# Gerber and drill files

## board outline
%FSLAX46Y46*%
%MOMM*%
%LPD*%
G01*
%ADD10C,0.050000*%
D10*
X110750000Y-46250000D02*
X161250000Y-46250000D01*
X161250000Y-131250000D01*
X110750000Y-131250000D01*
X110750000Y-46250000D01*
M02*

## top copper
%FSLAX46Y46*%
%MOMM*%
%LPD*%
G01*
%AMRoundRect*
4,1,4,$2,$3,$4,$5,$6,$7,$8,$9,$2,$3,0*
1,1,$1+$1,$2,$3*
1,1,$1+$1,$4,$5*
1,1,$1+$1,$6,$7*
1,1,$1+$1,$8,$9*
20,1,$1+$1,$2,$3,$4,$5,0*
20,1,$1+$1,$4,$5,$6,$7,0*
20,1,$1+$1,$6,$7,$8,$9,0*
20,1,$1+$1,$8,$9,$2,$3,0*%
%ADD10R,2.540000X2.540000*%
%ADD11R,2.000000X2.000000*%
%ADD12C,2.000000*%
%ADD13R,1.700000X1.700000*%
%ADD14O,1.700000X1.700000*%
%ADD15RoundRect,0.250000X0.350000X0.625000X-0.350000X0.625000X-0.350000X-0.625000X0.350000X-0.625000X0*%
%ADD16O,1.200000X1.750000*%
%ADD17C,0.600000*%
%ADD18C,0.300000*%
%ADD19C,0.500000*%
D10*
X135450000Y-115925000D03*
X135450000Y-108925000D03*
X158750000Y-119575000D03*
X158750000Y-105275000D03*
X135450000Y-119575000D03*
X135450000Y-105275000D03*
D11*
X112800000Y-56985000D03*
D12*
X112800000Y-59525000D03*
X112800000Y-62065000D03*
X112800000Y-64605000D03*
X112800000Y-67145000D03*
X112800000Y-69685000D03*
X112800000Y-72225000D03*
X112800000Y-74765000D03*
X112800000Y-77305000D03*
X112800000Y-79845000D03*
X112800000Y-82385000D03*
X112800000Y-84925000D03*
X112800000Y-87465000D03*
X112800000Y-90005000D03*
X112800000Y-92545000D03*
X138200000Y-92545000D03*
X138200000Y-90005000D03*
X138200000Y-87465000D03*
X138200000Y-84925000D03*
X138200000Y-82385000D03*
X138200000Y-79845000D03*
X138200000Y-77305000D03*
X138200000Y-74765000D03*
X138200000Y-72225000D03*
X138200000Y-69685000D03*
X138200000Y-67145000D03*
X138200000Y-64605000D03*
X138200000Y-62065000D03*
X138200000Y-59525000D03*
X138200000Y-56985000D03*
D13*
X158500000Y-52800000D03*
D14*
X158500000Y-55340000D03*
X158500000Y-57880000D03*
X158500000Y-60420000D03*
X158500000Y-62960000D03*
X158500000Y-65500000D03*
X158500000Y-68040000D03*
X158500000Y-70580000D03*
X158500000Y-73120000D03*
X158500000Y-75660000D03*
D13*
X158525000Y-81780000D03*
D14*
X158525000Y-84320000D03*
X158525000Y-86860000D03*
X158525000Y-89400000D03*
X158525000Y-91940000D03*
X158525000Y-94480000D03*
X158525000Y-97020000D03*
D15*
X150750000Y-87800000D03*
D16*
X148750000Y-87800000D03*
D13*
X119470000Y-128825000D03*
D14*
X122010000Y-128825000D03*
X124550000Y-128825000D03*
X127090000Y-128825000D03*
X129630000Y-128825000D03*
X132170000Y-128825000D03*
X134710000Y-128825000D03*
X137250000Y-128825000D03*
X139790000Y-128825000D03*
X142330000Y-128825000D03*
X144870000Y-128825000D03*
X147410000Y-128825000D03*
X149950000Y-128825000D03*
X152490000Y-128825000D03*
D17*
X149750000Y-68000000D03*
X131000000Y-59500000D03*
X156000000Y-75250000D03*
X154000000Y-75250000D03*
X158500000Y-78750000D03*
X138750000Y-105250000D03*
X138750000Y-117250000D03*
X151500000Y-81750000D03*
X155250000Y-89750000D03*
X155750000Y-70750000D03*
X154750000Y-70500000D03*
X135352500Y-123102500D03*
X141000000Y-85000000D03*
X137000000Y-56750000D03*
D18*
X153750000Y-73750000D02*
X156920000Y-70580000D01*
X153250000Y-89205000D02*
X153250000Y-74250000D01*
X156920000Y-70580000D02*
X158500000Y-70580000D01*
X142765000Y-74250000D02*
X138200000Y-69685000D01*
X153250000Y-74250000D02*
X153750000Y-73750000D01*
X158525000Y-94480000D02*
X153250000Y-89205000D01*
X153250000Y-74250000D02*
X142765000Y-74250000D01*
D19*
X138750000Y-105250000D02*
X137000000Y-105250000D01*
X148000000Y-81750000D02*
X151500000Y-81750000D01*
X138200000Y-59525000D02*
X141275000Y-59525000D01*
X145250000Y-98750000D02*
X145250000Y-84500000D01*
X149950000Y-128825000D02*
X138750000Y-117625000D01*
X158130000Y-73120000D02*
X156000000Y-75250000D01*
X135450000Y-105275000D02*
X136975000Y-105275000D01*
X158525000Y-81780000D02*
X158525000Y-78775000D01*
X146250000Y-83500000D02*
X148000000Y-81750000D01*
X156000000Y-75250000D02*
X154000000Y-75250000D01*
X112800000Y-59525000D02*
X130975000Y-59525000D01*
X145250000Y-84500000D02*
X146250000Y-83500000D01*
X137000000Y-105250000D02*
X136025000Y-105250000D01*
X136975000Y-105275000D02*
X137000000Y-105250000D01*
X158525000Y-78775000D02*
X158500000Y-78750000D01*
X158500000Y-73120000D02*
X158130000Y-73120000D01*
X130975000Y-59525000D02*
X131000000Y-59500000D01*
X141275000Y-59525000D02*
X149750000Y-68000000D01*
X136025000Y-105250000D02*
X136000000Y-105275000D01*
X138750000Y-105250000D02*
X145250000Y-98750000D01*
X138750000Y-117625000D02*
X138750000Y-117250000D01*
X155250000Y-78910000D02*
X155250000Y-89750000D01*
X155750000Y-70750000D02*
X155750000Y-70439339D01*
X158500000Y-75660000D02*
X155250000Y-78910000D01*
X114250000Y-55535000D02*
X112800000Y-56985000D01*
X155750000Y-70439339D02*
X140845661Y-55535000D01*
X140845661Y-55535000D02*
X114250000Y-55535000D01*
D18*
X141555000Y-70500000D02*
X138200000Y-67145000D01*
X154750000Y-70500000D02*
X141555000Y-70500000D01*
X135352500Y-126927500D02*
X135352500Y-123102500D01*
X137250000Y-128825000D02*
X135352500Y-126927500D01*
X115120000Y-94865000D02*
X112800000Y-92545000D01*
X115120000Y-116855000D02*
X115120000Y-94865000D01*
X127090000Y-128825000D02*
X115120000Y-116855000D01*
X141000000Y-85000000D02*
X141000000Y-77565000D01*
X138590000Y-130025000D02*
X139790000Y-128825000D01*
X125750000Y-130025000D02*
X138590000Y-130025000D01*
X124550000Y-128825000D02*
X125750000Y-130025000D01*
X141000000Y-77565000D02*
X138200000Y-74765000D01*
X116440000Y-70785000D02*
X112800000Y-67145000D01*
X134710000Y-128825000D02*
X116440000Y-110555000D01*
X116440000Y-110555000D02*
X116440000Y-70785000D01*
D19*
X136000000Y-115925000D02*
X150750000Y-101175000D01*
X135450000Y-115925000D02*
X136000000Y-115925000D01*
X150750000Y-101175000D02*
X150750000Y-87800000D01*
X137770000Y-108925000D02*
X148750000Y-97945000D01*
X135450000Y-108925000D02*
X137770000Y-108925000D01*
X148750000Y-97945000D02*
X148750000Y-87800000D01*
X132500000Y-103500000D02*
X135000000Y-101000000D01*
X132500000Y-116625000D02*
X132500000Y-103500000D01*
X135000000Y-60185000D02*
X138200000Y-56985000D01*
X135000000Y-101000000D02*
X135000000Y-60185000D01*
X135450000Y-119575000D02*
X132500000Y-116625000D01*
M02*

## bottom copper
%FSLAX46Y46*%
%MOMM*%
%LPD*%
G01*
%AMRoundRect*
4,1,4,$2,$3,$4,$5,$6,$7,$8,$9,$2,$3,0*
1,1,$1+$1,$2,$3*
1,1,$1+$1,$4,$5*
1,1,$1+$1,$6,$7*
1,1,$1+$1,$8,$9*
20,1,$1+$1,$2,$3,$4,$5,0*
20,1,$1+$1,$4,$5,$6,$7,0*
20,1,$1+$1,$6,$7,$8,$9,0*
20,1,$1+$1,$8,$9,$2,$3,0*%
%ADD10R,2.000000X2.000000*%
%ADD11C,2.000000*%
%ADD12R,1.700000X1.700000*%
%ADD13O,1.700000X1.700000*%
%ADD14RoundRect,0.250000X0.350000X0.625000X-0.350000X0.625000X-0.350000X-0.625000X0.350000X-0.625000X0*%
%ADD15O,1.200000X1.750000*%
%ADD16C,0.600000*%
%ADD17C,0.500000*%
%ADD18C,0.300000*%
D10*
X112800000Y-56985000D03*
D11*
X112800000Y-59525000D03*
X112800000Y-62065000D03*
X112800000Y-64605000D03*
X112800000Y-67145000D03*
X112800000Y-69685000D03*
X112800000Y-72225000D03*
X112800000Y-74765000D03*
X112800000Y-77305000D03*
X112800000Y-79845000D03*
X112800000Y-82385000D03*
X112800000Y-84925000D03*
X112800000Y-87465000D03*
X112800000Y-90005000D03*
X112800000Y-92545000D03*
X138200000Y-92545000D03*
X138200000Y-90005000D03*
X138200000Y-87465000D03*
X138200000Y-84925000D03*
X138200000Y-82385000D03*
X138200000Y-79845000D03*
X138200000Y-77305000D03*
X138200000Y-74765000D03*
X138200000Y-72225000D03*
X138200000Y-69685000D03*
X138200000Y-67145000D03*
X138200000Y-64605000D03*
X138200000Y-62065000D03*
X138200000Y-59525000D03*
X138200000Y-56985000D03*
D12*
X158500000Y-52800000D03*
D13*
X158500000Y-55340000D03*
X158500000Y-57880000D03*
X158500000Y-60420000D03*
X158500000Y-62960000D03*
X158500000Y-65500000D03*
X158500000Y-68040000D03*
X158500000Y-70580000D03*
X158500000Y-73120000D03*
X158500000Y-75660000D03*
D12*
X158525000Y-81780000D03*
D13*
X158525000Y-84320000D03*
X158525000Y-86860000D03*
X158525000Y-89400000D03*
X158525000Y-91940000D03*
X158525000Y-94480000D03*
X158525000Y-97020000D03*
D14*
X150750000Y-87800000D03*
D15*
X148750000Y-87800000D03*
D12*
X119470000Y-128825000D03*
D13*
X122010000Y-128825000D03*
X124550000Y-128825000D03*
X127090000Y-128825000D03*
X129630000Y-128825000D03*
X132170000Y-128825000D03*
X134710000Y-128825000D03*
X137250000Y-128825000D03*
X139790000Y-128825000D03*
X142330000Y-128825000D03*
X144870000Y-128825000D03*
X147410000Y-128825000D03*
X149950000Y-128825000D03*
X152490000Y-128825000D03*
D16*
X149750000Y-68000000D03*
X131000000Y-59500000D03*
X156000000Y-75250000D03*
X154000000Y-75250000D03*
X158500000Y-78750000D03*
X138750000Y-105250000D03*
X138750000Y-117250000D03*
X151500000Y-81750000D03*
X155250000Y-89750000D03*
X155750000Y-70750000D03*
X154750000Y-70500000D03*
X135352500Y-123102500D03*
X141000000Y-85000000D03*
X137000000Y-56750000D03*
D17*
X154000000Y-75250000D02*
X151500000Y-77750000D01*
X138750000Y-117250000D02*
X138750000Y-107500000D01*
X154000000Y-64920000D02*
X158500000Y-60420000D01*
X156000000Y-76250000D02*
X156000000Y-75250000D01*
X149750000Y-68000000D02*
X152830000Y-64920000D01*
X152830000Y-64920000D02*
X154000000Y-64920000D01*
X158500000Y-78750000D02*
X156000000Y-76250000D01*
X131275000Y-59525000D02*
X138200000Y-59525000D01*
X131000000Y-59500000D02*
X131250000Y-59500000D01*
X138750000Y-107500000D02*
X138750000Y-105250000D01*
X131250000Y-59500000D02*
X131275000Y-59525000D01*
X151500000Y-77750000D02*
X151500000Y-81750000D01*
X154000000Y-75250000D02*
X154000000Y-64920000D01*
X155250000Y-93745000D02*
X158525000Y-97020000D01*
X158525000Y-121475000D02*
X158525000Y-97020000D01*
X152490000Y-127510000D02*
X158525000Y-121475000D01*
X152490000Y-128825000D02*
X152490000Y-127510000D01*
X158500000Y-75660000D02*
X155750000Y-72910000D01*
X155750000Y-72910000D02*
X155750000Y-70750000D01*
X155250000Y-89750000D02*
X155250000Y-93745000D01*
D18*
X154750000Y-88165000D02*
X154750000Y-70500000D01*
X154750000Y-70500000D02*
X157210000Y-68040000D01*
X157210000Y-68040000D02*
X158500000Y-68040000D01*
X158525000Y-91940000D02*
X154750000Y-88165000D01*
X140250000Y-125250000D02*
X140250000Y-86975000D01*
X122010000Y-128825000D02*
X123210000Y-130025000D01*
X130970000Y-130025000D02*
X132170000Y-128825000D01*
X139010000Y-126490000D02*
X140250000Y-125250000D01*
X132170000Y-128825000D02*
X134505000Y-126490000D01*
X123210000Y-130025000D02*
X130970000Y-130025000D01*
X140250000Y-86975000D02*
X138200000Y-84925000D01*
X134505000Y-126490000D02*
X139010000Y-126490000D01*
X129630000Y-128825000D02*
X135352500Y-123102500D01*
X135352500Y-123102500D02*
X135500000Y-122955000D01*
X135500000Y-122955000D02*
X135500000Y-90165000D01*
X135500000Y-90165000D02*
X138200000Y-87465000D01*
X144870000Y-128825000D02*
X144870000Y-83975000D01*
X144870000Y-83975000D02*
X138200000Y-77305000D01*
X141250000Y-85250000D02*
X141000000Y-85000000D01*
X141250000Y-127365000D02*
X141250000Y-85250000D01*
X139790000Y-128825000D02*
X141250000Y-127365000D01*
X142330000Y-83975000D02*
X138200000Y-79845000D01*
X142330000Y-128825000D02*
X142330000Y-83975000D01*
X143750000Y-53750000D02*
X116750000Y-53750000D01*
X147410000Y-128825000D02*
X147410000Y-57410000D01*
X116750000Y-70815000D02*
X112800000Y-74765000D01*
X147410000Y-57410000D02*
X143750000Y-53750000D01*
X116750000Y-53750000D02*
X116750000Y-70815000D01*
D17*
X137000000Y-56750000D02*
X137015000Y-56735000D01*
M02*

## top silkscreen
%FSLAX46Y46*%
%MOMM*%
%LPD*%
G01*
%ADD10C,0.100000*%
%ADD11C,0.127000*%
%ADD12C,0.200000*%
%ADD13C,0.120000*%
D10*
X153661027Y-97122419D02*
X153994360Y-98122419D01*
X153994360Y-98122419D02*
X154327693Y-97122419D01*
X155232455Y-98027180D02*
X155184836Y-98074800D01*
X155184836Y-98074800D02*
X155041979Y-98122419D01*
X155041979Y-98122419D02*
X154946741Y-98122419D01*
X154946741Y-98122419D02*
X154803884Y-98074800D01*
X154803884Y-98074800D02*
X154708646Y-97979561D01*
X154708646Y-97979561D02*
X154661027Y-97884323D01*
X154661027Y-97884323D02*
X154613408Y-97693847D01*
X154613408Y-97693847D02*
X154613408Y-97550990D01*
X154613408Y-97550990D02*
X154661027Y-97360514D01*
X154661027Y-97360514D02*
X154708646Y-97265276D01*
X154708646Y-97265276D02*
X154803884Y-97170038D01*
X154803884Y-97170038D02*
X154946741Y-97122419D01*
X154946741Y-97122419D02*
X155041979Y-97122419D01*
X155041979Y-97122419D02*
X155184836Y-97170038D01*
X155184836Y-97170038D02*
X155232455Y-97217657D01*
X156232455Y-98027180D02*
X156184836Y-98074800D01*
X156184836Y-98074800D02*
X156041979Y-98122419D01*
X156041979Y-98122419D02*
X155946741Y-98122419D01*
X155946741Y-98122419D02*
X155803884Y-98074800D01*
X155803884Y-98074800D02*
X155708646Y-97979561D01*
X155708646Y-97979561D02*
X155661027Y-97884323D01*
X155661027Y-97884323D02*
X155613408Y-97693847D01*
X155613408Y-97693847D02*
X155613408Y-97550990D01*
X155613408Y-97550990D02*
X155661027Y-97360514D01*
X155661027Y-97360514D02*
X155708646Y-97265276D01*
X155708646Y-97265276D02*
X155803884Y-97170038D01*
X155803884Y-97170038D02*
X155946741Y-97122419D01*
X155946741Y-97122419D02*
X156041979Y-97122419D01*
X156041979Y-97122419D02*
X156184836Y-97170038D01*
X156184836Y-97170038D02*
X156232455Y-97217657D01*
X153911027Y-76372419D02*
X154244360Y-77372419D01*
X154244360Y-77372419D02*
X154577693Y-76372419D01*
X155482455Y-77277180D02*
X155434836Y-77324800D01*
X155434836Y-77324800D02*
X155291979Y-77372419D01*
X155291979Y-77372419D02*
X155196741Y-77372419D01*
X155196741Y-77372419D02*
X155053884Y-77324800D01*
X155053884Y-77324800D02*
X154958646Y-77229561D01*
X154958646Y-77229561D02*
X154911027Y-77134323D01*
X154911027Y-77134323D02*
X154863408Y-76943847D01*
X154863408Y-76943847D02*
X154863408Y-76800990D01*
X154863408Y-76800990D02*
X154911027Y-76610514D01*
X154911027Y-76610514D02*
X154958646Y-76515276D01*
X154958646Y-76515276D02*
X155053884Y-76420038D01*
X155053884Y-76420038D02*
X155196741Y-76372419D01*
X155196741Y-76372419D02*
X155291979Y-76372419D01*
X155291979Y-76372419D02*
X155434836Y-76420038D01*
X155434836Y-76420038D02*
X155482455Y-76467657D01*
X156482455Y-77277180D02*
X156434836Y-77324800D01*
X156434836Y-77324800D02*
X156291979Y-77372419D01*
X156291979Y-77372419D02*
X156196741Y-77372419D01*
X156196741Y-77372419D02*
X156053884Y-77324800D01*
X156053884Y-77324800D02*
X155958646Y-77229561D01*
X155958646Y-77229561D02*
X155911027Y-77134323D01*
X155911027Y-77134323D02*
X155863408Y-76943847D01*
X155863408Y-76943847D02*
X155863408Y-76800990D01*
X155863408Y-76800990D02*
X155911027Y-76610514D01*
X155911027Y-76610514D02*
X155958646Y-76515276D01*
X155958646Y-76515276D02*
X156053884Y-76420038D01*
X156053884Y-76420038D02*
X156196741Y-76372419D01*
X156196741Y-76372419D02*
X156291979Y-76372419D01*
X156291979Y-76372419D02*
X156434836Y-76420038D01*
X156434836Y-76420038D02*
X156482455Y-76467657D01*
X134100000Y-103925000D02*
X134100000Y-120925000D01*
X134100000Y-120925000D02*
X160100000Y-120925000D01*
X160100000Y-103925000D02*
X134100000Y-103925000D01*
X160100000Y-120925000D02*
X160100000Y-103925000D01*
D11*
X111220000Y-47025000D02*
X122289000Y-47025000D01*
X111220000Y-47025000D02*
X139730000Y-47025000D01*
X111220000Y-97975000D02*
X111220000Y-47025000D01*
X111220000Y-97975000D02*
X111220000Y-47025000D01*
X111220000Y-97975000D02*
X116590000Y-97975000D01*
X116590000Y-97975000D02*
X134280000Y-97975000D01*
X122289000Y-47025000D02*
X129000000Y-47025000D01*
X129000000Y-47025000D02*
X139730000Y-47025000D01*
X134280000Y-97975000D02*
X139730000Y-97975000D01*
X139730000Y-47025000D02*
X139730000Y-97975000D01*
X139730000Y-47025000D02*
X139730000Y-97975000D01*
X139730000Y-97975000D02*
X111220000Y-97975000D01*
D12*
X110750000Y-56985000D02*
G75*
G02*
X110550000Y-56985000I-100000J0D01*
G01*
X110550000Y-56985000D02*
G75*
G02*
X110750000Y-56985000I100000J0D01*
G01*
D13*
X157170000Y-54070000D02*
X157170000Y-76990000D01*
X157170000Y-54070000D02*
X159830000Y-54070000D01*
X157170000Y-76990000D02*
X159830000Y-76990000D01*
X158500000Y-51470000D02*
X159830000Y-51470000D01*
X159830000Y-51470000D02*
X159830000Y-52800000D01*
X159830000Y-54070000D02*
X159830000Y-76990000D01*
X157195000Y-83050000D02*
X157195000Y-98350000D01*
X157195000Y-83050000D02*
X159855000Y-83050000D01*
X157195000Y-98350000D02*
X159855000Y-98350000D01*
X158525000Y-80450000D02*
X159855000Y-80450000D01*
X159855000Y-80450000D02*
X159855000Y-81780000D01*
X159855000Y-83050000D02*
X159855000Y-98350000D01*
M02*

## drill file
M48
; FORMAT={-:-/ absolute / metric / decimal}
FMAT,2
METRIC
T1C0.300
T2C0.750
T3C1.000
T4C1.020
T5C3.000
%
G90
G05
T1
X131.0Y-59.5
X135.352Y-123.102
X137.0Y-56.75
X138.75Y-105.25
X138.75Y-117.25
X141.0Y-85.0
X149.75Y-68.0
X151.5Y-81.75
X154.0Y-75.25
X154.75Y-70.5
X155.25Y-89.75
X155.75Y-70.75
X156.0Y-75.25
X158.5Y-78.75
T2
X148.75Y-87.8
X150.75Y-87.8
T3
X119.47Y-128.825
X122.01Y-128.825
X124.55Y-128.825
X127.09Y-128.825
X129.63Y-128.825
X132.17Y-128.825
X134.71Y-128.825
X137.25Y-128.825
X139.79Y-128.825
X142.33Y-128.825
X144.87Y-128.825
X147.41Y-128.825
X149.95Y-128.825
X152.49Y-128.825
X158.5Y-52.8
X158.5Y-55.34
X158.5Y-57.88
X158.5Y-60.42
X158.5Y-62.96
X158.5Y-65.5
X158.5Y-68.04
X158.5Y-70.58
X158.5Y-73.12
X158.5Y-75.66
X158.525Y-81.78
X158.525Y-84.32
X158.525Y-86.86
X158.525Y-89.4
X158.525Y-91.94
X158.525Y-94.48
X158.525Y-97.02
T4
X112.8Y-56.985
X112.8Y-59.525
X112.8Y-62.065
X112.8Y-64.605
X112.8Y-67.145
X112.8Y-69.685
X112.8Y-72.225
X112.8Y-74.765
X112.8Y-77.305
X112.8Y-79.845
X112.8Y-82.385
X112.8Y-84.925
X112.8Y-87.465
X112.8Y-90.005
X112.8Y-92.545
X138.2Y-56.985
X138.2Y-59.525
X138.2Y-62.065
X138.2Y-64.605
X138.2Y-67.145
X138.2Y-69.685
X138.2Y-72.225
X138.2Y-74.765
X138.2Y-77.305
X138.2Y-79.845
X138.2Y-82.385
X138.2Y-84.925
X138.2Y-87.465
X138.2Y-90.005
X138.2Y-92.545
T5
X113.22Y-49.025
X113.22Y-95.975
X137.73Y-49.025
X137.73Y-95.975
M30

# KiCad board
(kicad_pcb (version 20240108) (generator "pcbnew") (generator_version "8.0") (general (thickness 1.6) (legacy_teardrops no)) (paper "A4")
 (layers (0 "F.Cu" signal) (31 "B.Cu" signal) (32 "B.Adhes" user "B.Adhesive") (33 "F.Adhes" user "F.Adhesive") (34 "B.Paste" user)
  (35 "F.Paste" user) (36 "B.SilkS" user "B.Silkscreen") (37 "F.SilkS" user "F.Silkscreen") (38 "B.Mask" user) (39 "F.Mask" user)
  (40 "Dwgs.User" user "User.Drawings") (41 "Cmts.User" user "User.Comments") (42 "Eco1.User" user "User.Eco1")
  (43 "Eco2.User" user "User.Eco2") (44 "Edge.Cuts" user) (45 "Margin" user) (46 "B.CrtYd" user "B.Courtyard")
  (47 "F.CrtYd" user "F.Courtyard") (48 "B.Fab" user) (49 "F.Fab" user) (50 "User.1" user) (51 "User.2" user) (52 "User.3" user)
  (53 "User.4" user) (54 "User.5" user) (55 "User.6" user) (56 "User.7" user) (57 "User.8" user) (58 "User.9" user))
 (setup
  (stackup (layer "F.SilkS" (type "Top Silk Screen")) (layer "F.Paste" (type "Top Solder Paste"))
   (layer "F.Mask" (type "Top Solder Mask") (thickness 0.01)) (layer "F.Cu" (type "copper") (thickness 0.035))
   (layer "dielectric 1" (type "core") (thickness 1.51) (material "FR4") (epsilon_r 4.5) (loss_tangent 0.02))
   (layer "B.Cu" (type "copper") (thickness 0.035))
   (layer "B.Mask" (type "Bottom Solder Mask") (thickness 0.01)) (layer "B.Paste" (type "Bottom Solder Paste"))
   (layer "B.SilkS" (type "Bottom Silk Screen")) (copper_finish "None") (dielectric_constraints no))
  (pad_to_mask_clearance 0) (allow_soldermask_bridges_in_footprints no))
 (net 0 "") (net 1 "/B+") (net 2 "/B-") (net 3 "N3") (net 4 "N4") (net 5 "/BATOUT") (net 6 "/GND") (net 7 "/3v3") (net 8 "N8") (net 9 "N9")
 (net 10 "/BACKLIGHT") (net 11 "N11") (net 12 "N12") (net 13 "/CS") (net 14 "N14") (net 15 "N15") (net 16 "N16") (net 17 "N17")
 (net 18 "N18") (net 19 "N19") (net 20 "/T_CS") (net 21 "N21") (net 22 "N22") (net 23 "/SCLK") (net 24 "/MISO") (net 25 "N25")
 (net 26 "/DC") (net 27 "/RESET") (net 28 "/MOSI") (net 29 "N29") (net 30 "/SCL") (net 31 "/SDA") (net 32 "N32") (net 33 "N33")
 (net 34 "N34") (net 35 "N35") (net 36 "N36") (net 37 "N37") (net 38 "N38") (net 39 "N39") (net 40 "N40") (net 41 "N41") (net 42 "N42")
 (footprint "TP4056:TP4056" (layer "F.Cu") (at 134.1 103.925 -90)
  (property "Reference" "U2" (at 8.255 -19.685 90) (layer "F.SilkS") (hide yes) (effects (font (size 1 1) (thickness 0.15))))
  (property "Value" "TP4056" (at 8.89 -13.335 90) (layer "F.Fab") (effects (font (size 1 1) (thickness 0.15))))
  (fp_line (start 0 0) (end 17 0) (stroke (width 0.1) (type solid)) (layer "F.SilkS"))
  (fp_line (start 17 0) (end 17 -26) (stroke (width 0.1) (type solid)) (layer "F.SilkS"))
  (fp_line (start 0 -26) (end 0 0) (stroke (width 0.1) (type solid)) (layer "F.SilkS"))
  (fp_line (start 17 -26) (end 0 -26) (stroke (width 0.1) (type solid)) (layer "F.SilkS"))
  (pad "B+" smd rect (at 12 -1.35 270) (size 2.54 2.54) (layers "F.Cu" "F.Paste" "F.Mask") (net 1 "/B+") (solder_mask_margin 0.102))
  (pad "B-" smd rect (at 5 -1.35 270) (size 2.54 2.54) (layers "F.Cu" "F.Paste" "F.Mask") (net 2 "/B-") (solder_mask_margin 0.102))
  (pad "IN+" smd rect (at 15.65 -24.65 270) (size 2.54 2.54) (layers "F.Cu" "F.Paste" "F.Mask") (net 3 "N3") (solder_mask_margin 0.102))
  (pad "IN-" smd rect (at 1.35 -24.65 270) (size 2.54 2.54) (layers "F.Cu" "F.Paste" "F.Mask") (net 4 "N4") (solder_mask_margin 0.102))
  (pad "OUT+" smd rect (at 15.65 -1.35 270) (size 2.54 2.54) (layers "F.Cu" "F.Paste" "F.Mask") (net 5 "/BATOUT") (solder_mask_margin 0.102))
  (pad "OUT-" smd rect (at 1.35 -1.35 270) (size 2.54 2.54) (layers "F.Cu" "F.Paste" "F.Mask") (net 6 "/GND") (solder_mask_margin 0.102)))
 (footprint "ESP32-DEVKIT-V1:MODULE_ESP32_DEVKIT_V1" (layer "F.Cu") (at 125.5 72.5)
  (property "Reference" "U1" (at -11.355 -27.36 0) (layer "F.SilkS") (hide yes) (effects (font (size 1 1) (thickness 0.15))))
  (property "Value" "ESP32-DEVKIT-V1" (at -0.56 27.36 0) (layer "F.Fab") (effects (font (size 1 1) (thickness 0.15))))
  (fp_line (start -14.28 -25.475) (end -3.211 -25.475) (stroke (width 0.127) (type solid)) (layer "F.SilkS"))
  (fp_line (start -14.28 -25.475) (end 14.23 -25.475) (stroke (width 0.127) (type solid)) (layer "F.SilkS"))
  (fp_line (start -14.28 25.475) (end -14.28 -25.475) (stroke (width 0.127) (type solid)) (layer "F.SilkS"))
  (fp_line (start -14.28 25.475) (end -14.28 -25.475) (stroke (width 0.127) (type solid)) (layer "F.SilkS"))
  (fp_line (start -14.28 25.475) (end -8.91 25.475) (stroke (width 0.127) (type solid)) (layer "F.SilkS"))
  (fp_line (start -8.91 25.475) (end 8.78 25.475) (stroke (width 0.127) (type solid)) (layer "F.SilkS"))
  (fp_line (start -3.211 -25.475) (end 3.5 -25.475) (stroke (width 0.127) (type solid)) (layer "F.SilkS"))
  (fp_line (start 3.5 -25.475) (end 14.23 -25.475) (stroke (width 0.127) (type solid)) (layer "F.SilkS"))
  (fp_line (start 8.78 25.475) (end 14.23 25.475) (stroke (width 0.127) (type solid)) (layer "F.SilkS"))
  (fp_line (start 14.23 -25.475) (end 14.23 25.475) (stroke (width 0.127) (type solid)) (layer "F.SilkS"))
  (fp_line (start 14.23 -25.475) (end 14.23 25.475) (stroke (width 0.127) (type solid)) (layer "F.SilkS"))
  (fp_line (start 14.23 25.475) (end -14.28 25.475) (stroke (width 0.127) (type solid)) (layer "F.SilkS"))
  (fp_circle (center -14.85 -15.515) (end -14.75 -15.515) (stroke (width 0.2) (type solid)) (fill none) (layer "F.SilkS"))
  (pad "" np_thru_hole circle (at -12.28 -23.475) (size 3 3) (drill 3) (layers "*.Cu" "*.Mask"))
  (pad "" np_thru_hole circle (at -12.28 23.475) (size 3 3) (drill 3) (layers "*.Cu" "*.Mask"))
  (pad "" np_thru_hole circle (at 12.23 -23.475) (size 3 3) (drill 3) (layers "*.Cu" "*.Mask"))
  (pad "" np_thru_hole circle (at 12.23 23.475) (size 3 3) (drill 3) (layers "*.Cu" "*.Mask"))
  (pad "1" thru_hole rect (at -12.7 -15.515) (size 2 2) (drill 1.02) (layers "*.Cu" "*.Mask") (remove_unused_layers no) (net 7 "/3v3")
   (solder_mask_margin 0.102))
  (pad "2" thru_hole circle (at -12.7 -12.975) (size 2 2) (drill 1.02) (layers "*.Cu" "*.Mask") (remove_unused_layers no) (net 6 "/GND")
   (solder_mask_margin 0.102))
  (pad "3" thru_hole circle (at -12.7 -10.435) (size 2 2) (drill 1.02) (layers "*.Cu" "*.Mask") (remove_unused_layers no) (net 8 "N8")
   (solder_mask_margin 0.102))
  (pad "4" thru_hole circle (at -12.7 -7.895) (size 2 2) (drill 1.02) (layers "*.Cu" "*.Mask") (remove_unused_layers no) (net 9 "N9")
   (solder_mask_margin 0.102))
  (pad "5" thru_hole circle (at -12.7 -5.355) (size 2 2) (drill 1.02) (layers "*.Cu" "*.Mask") (remove_unused_layers no)
   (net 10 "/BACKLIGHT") (solder_mask_margin 0.102))
  (pad "6" thru_hole circle (at -12.7 -2.815) (size 2 2) (drill 1.02) (layers "*.Cu" "*.Mask") (remove_unused_layers no) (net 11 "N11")
   (solder_mask_margin 0.102))
  (pad "7" thru_hole circle (at -12.7 -0.275) (size 2 2) (drill 1.02) (layers "*.Cu" "*.Mask") (remove_unused_layers no) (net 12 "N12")
   (solder_mask_margin 0.102))
  (pad "8" thru_hole circle (at -12.7 2.265) (size 2 2) (drill 1.02) (layers "*.Cu" "*.Mask") (remove_unused_layers no) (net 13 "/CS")
   (solder_mask_margin 0.102))
  (pad "9" thru_hole circle (at -12.7 4.805) (size 2 2) (drill 1.02) (layers "*.Cu" "*.Mask") (remove_unused_layers no) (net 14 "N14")
   (solder_mask_margin 0.102))
  (pad "10" thru_hole circle (at -12.7 7.345) (size 2 2) (drill 1.02) (layers "*.Cu" "*.Mask") (remove_unused_layers no) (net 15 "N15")
   (solder_mask_margin 0.102))
  (pad "11" thru_hole circle (at -12.7 9.885) (size 2 2) (drill 1.02) (layers "*.Cu" "*.Mask") (remove_unused_layers no) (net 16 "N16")
   (solder_mask_margin 0.102))
  (pad "12" thru_hole circle (at -12.7 12.425) (size 2 2) (drill 1.02) (layers "*.Cu" "*.Mask") (remove_unused_layers no) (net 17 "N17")
   (solder_mask_margin 0.102))
  (pad "13" thru_hole circle (at -12.7 14.965) (size 2 2) (drill 1.02) (layers "*.Cu" "*.Mask") (remove_unused_layers no) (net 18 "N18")
   (solder_mask_margin 0.102))
  (pad "14" thru_hole circle (at -12.7 17.505) (size 2 2) (drill 1.02) (layers "*.Cu" "*.Mask") (remove_unused_layers no) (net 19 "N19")
   (solder_mask_margin 0.102))
  (pad "15" thru_hole circle (at -12.7 20.045) (size 2 2) (drill 1.02) (layers "*.Cu" "*.Mask") (remove_unused_layers no) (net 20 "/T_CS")
   (solder_mask_margin 0.102))
  (pad "16" thru_hole circle (at 12.7 20.045) (size 2 2) (drill 1.02) (layers "*.Cu" "*.Mask") (remove_unused_layers no) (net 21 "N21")
   (solder_mask_margin 0.102))
  (pad "17" thru_hole circle (at 12.7 17.505) (size 2 2) (drill 1.02) (layers "*.Cu" "*.Mask") (remove_unused_layers no) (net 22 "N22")
   (solder_mask_margin 0.102))
  (pad "18" thru_hole circle (at 12.7 14.965) (size 2 2) (drill 1.02) (layers "*.Cu" "*.Mask") (remove_unused_layers no) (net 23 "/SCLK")
   (solder_mask_margin 0.102))
  (pad "19" thru_hole circle (at 12.7 12.425) (size 2 2) (drill 1.02) (layers "*.Cu" "*.Mask") (remove_unused_layers no) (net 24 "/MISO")
   (solder_mask_margin 0.102))
  (pad "20" thru_hole circle (at 12.7 9.885) (size 2 2) (drill 1.02) (layers "*.Cu" "*.Mask") (remove_unused_layers no) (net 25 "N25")
   (solder_mask_margin 0.102))
  (pad "21" thru_hole circle (at 12.7 7.345) (size 2 2) (drill 1.02) (layers "*.Cu" "*.Mask") (remove_unused_layers no) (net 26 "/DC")
   (solder_mask_margin 0.102))
  (pad "22" thru_hole circle (at 12.7 4.805) (size 2 2) (drill 1.02) (layers "*.Cu" "*.Mask") (remove_unused_layers no) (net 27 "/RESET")
   (solder_mask_margin 0.102))
  (pad "23" thru_hole circle (at 12.7 2.265) (size 2 2) (drill 1.02) (layers "*.Cu" "*.Mask") (remove_unused_layers no) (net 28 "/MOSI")
   (solder_mask_margin 0.102))
  (pad "24" thru_hole circle (at 12.7 -0.275) (size 2 2) (drill 1.02) (layers "*.Cu" "*.Mask") (remove_unused_layers no) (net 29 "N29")
   (solder_mask_margin 0.102))
  (pad "25" thru_hole circle (at 12.7 -2.815) (size 2 2) (drill 1.02) (layers "*.Cu" "*.Mask") (remove_unused_layers no) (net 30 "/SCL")
   (solder_mask_margin 0.102))
  (pad "26" thru_hole circle (at 12.7 -5.355) (size 2 2) (drill 1.02) (layers "*.Cu" "*.Mask") (remove_unused_layers no) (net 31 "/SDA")
   (solder_mask_margin 0.102))
  (pad "27" thru_hole circle (at 12.7 -7.895) (size 2 2) (drill 1.02) (layers "*.Cu" "*.Mask") (remove_unused_layers no) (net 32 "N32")
   (solder_mask_margin 0.102))
  (pad "28" thru_hole circle (at 12.7 -10.435) (size 2 2) (drill 1.02) (layers "*.Cu" "*.Mask") (remove_unused_layers no) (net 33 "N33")
   (solder_mask_margin 0.102))
  (pad "29" thru_hole circle (at 12.7 -12.975) (size 2 2) (drill 1.02) (layers "*.Cu" "*.Mask") (remove_unused_layers no) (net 6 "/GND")
   (solder_mask_margin 0.102))
  (pad "30" thru_hole circle (at 12.7 -15.515) (size 2 2) (drill 1.02) (layers "*.Cu" "*.Mask") (remove_unused_layers no) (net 5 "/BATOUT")
   (solder_mask_margin 0.102))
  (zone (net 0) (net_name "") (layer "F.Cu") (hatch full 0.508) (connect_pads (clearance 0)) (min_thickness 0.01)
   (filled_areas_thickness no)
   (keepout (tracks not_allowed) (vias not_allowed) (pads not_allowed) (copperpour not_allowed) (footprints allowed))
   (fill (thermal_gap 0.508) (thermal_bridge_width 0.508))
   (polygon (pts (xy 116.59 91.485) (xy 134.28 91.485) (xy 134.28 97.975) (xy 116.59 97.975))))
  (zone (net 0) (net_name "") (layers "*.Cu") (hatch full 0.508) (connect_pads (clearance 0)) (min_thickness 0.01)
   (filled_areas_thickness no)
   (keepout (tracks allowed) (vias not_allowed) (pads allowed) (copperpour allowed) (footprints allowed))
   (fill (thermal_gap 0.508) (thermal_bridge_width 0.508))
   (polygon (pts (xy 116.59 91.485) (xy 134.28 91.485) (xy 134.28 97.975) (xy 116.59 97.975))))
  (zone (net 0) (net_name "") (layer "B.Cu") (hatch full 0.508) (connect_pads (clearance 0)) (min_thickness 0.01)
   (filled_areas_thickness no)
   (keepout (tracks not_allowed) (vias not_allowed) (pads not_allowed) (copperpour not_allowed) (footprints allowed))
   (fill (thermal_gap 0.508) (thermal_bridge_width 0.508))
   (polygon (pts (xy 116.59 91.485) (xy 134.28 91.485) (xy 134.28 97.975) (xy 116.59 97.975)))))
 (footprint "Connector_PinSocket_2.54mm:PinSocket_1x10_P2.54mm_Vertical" (layer "F.Cu") (at 158.5 52.8)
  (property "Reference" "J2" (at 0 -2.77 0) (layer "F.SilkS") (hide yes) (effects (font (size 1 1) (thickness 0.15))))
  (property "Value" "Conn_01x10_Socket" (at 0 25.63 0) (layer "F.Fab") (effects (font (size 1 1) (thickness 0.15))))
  (fp_line (start -1.33 1.27) (end -1.33 24.19) (stroke (width 0.12) (type solid)) (layer "F.SilkS"))
  (fp_line (start -1.33 1.27) (end 1.33 1.27) (stroke (width 0.12) (type solid)) (layer "F.SilkS"))
  (fp_line (start -1.33 24.19) (end 1.33 24.19) (stroke (width 0.12) (type solid)) (layer "F.SilkS"))
  (fp_line (start 0 -1.33) (end 1.33 -1.33) (stroke (width 0.12) (type solid)) (layer "F.SilkS"))
  (fp_line (start 1.33 -1.33) (end 1.33 0) (stroke (width 0.12) (type solid)) (layer "F.SilkS"))
  (fp_line (start 1.33 1.27) (end 1.33 24.19) (stroke (width 0.12) (type solid)) (layer "F.SilkS"))
  (pad "1" thru_hole rect (at 0 0) (size 1.7 1.7) (drill 1) (layers "*.Cu" "*.Mask") (remove_unused_layers no) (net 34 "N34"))
  (pad "2" thru_hole oval (at 0 2.54) (size 1.7 1.7) (drill 1) (layers "*.Cu" "*.Mask") (remove_unused_layers no) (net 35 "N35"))
  (pad "3" thru_hole oval (at 0 5.08) (size 1.7 1.7) (drill 1) (layers "*.Cu" "*.Mask") (remove_unused_layers no) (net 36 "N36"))
  (pad "4" thru_hole oval (at 0 7.62) (size 1.7 1.7) (drill 1) (layers "*.Cu" "*.Mask") (remove_unused_layers no) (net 6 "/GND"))
  (pad "5" thru_hole oval (at 0 10.16) (size 1.7 1.7) (drill 1) (layers "*.Cu" "*.Mask") (remove_unused_layers no) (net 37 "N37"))
  (pad "6" thru_hole oval (at 0 12.7) (size 1.7 1.7) (drill 1) (layers "*.Cu" "*.Mask") (remove_unused_layers no) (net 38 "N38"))
  (pad "7" thru_hole oval (at 0 15.24) (size 1.7 1.7) (drill 1) (layers "*.Cu" "*.Mask") (remove_unused_layers no) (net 31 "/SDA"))
  (pad "8" thru_hole oval (at 0 17.78) (size 1.7 1.7) (drill 1) (layers "*.Cu" "*.Mask") (remove_unused_layers no) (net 30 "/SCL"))
  (pad "9" thru_hole oval (at 0 20.32) (size 1.7 1.7) (drill 1) (layers "*.Cu" "*.Mask") (remove_unused_layers no) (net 6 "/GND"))
  (pad "10" thru_hole oval (at 0 22.86) (size 1.7 1.7) (drill 1) (layers "*.Cu" "*.Mask") (remove_unused_layers no) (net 7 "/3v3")))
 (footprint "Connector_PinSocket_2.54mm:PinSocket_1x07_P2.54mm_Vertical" (layer "F.Cu") (at 158.525 81.78)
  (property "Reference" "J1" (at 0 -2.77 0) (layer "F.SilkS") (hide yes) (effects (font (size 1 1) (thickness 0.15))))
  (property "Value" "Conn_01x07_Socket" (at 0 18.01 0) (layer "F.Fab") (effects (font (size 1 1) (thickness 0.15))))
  (fp_line (start -1.33 1.27) (end -1.33 16.57) (stroke (width 0.12) (type solid)) (layer "F.SilkS"))
  (fp_line (start -1.33 1.27) (end 1.33 1.27) (stroke (width 0.12) (type solid)) (layer "F.SilkS"))
  (fp_line (start -1.33 16.57) (end 1.33 16.57) (stroke (width 0.12) (type solid)) (layer "F.SilkS"))
  (fp_line (start 0 -1.33) (end 1.33 -1.33) (stroke (width 0.12) (type solid)) (layer "F.SilkS"))
  (fp_line (start 1.33 -1.33) (end 1.33 0) (stroke (width 0.12) (type solid)) (layer "F.SilkS"))
  (fp_line (start 1.33 1.27) (end 1.33 16.57) (stroke (width 0.12) (type solid)) (layer "F.SilkS"))
  (pad "1" thru_hole rect (at 0 0) (size 1.7 1.7) (drill 1) (layers "*.Cu" "*.Mask") (remove_unused_layers no) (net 6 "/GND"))
  (pad "2" thru_hole oval (at 0 2.54) (size 1.7 1.7) (drill 1) (layers "*.Cu" "*.Mask") (remove_unused_layers no) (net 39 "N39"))
  (pad "3" thru_hole oval (at 0 5.08) (size 1.7 1.7) (drill 1) (layers "*.Cu" "*.Mask") (remove_unused_layers no) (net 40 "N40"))
  (pad "4" thru_hole oval (at 0 7.62) (size 1.7 1.7) (drill 1) (layers "*.Cu" "*.Mask") (remove_unused_layers no) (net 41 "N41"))
  (pad "5" thru_hole oval (at 0 10.16) (size 1.7 1.7) (drill 1) (layers "*.Cu" "*.Mask") (remove_unused_layers no) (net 31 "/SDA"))
  (pad "6" thru_hole oval (at 0 12.7) (size 1.7 1.7) (drill 1) (layers "*.Cu" "*.Mask") (remove_unused_layers no) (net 30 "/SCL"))
  (pad "7" thru_hole oval (at 0 15.24) (size 1.7 1.7) (drill 1) (layers "*.Cu" "*.Mask") (remove_unused_layers no) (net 7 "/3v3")))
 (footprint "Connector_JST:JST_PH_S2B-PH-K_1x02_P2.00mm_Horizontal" (layer "B.Cu") (at 150.75 87.8 180)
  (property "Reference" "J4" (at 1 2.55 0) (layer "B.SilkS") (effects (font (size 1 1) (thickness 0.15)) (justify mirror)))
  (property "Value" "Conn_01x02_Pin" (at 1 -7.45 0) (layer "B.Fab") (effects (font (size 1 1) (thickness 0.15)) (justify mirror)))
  (pad "1" thru_hole roundrect (at 0 0 180) (size 1.2 1.75) (drill 0.75) (layers "*.Cu" "*.Mask") (remove_unused_layers no)
   (roundrect_rratio 0.208333) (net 1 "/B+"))
  (pad "2" thru_hole oval (at 2 0 180) (size 1.2 1.75) (drill 0.75) (layers "*.Cu" "*.Mask") (remove_unused_layers no) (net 2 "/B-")))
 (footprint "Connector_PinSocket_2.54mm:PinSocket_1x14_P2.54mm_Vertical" (layer "B.Cu") (at 119.47 128.825 -90)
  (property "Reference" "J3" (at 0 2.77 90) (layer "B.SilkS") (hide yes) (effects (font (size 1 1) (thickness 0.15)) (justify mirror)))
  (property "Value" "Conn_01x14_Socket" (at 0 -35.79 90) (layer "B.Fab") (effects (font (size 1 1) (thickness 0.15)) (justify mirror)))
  (pad "1" thru_hole rect (at 0 0 270) (size 1.7 1.7) (drill 1) (layers "*.Cu" "*.Mask") (remove_unused_layers no) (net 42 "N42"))
  (pad "2" thru_hole oval (at 0 -2.54 270) (size 1.7 1.7) (drill 1) (layers "*.Cu" "*.Mask") (remove_unused_layers no) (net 24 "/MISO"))
  (pad "3" thru_hole oval (at 0 -5.08 270) (size 1.7 1.7) (drill 1) (layers "*.Cu" "*.Mask") (remove_unused_layers no) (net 28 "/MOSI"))
  (pad "4" thru_hole oval (at 0 -7.62 270) (size 1.7 1.7) (drill 1) (layers "*.Cu" "*.Mask") (remove_unused_layers no) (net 20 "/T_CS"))
  (pad "5" thru_hole oval (at 0 -10.16 270) (size 1.7 1.7) (drill 1) (layers "*.Cu" "*.Mask") (remove_unused_layers no) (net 23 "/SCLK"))
  (pad "6" thru_hole oval (at 0 -12.7 270) (size 1.7 1.7) (drill 1) (layers "*.Cu" "*.Mask") (remove_unused_layers no) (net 24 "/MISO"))
  (pad "7" thru_hole oval (at 0 -15.24 270) (size 1.7 1.7) (drill 1) (layers "*.Cu" "*.Mask") (remove_unused_layers no)
   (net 10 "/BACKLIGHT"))
  (pad "8" thru_hole oval (at 0 -17.78 270) (size 1.7 1.7) (drill 1) (layers "*.Cu" "*.Mask") (remove_unused_layers no) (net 23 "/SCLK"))
  (pad "9" thru_hole oval (at 0 -20.32 270) (size 1.7 1.7) (drill 1) (layers "*.Cu" "*.Mask") (remove_unused_layers no) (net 28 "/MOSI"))
  (pad "10" thru_hole oval (at 0 -22.86 270) (size 1.7 1.7) (drill 1) (layers "*.Cu" "*.Mask") (remove_unused_layers no) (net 26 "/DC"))
  (pad "11" thru_hole oval (at 0 -25.4 270) (size 1.7 1.7) (drill 1) (layers "*.Cu" "*.Mask") (remove_unused_layers no) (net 27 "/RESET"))
  (pad "12" thru_hole oval (at 0 -27.94 270) (size 1.7 1.7) (drill 1) (layers "*.Cu" "*.Mask") (remove_unused_layers no) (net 13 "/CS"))
  (pad "13" thru_hole oval (at 0 -30.48 270) (size 1.7 1.7) (drill 1) (layers "*.Cu" "*.Mask") (remove_unused_layers no) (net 6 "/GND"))
  (pad "14" thru_hole oval (at 0 -33.02 270) (size 1.7 1.7) (drill 1) (layers "*.Cu" "*.Mask") (remove_unused_layers no) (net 7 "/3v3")))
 (gr_rect (start 110.75 46.25) (end 161.25 131.25) (stroke (width 0.05) (type default)) (fill none) (layer "Edge.Cuts"))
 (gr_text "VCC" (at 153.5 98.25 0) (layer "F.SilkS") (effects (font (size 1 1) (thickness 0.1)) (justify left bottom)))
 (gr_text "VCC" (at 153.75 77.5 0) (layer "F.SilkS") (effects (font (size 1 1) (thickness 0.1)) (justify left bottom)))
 (segment (start 153.75 73.75) (end 156.92 70.58) (width 0.3) (layer "F.Cu") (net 30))
 (segment (start 153.25 89.205) (end 153.25 74.25) (width 0.3) (layer "F.Cu") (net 30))
 (segment (start 156.92 70.58) (end 158.5 70.58) (width 0.3) (layer "F.Cu") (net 30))
 (segment (start 142.765 74.25) (end 138.2 69.685) (width 0.3) (layer "F.Cu") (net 30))
 (segment (start 153.25 74.25) (end 153.75 73.75) (width 0.3) (layer "F.Cu") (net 30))
 (segment (start 158.525 94.48) (end 153.25 89.205) (width 0.3) (layer "F.Cu") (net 30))
 (segment (start 153.25 74.25) (end 142.765 74.25) (width 0.3) (layer "F.Cu") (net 30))
 (segment (start 138.75 105.25) (end 137 105.25) (width 0.5) (layer "F.Cu") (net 6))
 (segment (start 148 81.75) (end 151.5 81.75) (width 0.5) (layer "F.Cu") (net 6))
 (segment (start 138.2 59.525) (end 141.275 59.525) (width 0.5) (layer "F.Cu") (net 6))
 (segment (start 145.25 98.75) (end 145.25 84.5) (width 0.5) (layer "F.Cu") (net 6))
 (segment (start 149.95 128.825) (end 138.75 117.625) (width 0.5) (layer "F.Cu") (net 6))
 (segment (start 158.13 73.12) (end 156 75.25) (width 0.5) (layer "F.Cu") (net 6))
 (segment (start 135.45 105.275) (end 136.975 105.275) (width 0.5) (layer "F.Cu") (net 6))
 (segment (start 158.525 81.78) (end 158.525 78.775) (width 0.5) (layer "F.Cu") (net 6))
 (segment (start 146.25 83.5) (end 148 81.75) (width 0.5) (layer "F.Cu") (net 6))
 (segment (start 156 75.25) (end 154 75.25) (width 0.5) (layer "F.Cu") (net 6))
 (segment (start 112.8 59.525) (end 130.975 59.525) (width 0.5) (layer "F.Cu") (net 6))
 (segment (start 145.25 84.5) (end 146.25 83.5) (width 0.5) (layer "F.Cu") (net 6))
 (segment (start 137 105.25) (end 136.025 105.25) (width 0.5) (layer "F.Cu") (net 6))
 (segment (start 136.975 105.275) (end 137 105.25) (width 0.5) (layer "F.Cu") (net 6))
 (segment (start 158.525 78.775) (end 158.5 78.75) (width 0.5) (layer "F.Cu") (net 6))
 (segment (start 158.5 73.12) (end 158.13 73.12) (width 0.5) (layer "F.Cu") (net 6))
 (segment (start 130.975 59.525) (end 131 59.5) (width 0.5) (layer "F.Cu") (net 6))
 (segment (start 141.275 59.525) (end 149.75 68) (width 0.5) (layer "F.Cu") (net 6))
 (segment (start 136.025 105.25) (end 136 105.275) (width 0.5) (layer "F.Cu") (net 6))
 (segment (start 138.75 105.25) (end 145.25 98.75) (width 0.5) (layer "F.Cu") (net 6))
 (segment (start 138.75 117.625) (end 138.75 117.25) (width 0.5) (layer "F.Cu") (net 6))
 (via (at 149.75 68) (size 0.6) (drill 0.3) (layers "F.Cu" "B.Cu") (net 6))
 (via (at 131 59.5) (size 0.6) (drill 0.3) (layers "F.Cu" "B.Cu") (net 6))
 (via (at 156 75.25) (size 0.6) (drill 0.3) (layers "F.Cu" "B.Cu") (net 6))
 (via (at 154 75.25) (size 0.6) (drill 0.3) (layers "F.Cu" "B.Cu") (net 6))
 (via (at 158.5 78.75) (size 0.6) (drill 0.3) (layers "F.Cu" "B.Cu") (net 6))
 (via (at 138.75 105.25) (size 0.6) (drill 0.3) (layers "F.Cu" "B.Cu") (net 6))
 (via (at 138.75 117.25) (size 0.6) (drill 0.3) (layers "F.Cu" "B.Cu") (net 6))
 (via (at 151.5 81.75) (size 0.6) (drill 0.3) (layers "F.Cu" "B.Cu") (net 6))
 (segment (start 154 75.25) (end 151.5 77.75) (width 0.5) (layer "B.Cu") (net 6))
 (segment (start 138.75 117.25) (end 138.75 107.5) (width 0.5) (layer "B.Cu") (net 6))
 (segment (start 154 64.92) (end 158.5 60.42) (width 0.5) (layer "B.Cu") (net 6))
 (segment (start 156 76.25) (end 156 75.25) (width 0.5) (layer "B.Cu") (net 6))
 (segment (start 149.75 68) (end 152.83 64.92) (width 0.5) (layer "B.Cu") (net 6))
 (segment (start 152.83 64.92) (end 154 64.92) (width 0.5) (layer "B.Cu") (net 6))
 (segment (start 158.5 78.75) (end 156 76.25) (width 0.5) (layer "B.Cu") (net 6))
 (segment (start 131.275 59.525) (end 138.2 59.525) (width 0.5) (layer "B.Cu") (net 6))
 (segment (start 131 59.5) (end 131.25 59.5) (width 0.5) (layer "B.Cu") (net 6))
 (segment (start 138.75 107.5) (end 138.75 105.25) (width 0.5) (layer "B.Cu") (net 6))
 (segment (start 131.25 59.5) (end 131.275 59.525) (width 0.5) (layer "B.Cu") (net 6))
 (segment (start 151.5 77.75) (end 151.5 81.75) (width 0.5) (layer "B.Cu") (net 6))
 (segment (start 154 75.25) (end 154 64.92) (width 0.5) (layer "B.Cu") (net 6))
 (segment (start 155.25 78.91) (end 155.25 89.75) (width 0.5) (layer "F.Cu") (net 7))
 (segment (start 155.75 70.75) (end 155.75 70.439339) (width 0.5) (layer "F.Cu") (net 7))
 (segment (start 158.5 75.66) (end 155.25 78.91) (width 0.5) (layer "F.Cu") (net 7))
 (segment (start 114.25 55.535) (end 112.8 56.985) (width 0.5) (layer "F.Cu") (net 7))
 (segment (start 155.75 70.439339) (end 140.845661 55.535) (width 0.5) (layer "F.Cu") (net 7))
 (segment (start 140.845661 55.535) (end 114.25 55.535) (width 0.5) (layer "F.Cu") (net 7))
 (via (at 155.25 89.75) (size 0.6) (drill 0.3) (layers "F.Cu" "B.Cu") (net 7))
 (via (at 155.75 70.75) (size 0.6) (drill 0.3) (layers "F.Cu" "B.Cu") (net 7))
 (segment (start 155.25 93.745) (end 158.525 97.02) (width 0.5) (layer "B.Cu") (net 7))
 (segment (start 158.525 121.475) (end 158.525 97.02) (width 0.5) (layer "B.Cu") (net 7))
 (segment (start 152.49 127.51) (end 158.525 121.475) (width 0.5) (layer "B.Cu") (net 7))
 (segment (start 152.49 128.825) (end 152.49 127.51) (width 0.5) (layer "B.Cu") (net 7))
 (segment (start 158.5 75.66) (end 155.75 72.91) (width 0.5) (layer "B.Cu") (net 7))
 (segment (start 155.75 72.91) (end 155.75 70.75) (width 0.5) (layer "B.Cu") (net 7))
 (segment (start 155.25 89.75) (end 155.25 93.745) (width 0.5) (layer "B.Cu") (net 7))
 (segment (start 141.555 70.5) (end 138.2 67.145) (width 0.3) (layer "F.Cu") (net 31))
 (segment (start 154.75 70.5) (end 141.555 70.5) (width 0.3) (layer "F.Cu") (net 31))
 (via (at 154.75 70.5) (size 0.6) (drill 0.3) (layers "F.Cu" "B.Cu") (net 31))
 (segment (start 154.75 88.165) (end 154.75 70.5) (width 0.3) (layer "B.Cu") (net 31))
 (segment (start 154.75 70.5) (end 157.21 68.04) (width 0.3) (layer "B.Cu") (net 31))
 (segment (start 157.21 68.04) (end 158.5 68.04) (width 0.3) (layer "B.Cu") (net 31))
 (segment (start 158.525 91.94) (end 154.75 88.165) (width 0.3) (layer "B.Cu") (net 31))
 (segment (start 140.25 125.25) (end 140.25 86.975) (width 0.3) (layer "B.Cu") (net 24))
 (segment (start 122.01 128.825) (end 123.21 130.025) (width 0.3) (layer "B.Cu") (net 24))
 (segment (start 130.97 130.025) (end 132.17 128.825) (width 0.3) (layer "B.Cu") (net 24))
 (segment (start 139.01 126.49) (end 140.25 125.25) (width 0.3) (layer "B.Cu") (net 24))
 (segment (start 132.17 128.825) (end 134.505 126.49) (width 0.3) (layer "B.Cu") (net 24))
 (segment (start 123.21 130.025) (end 130.97 130.025) (width 0.3) (layer "B.Cu") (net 24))
 (segment (start 140.25 86.975) (end 138.2 84.925) (width 0.3) (layer "B.Cu") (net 24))
 (segment (start 134.505 126.49) (end 139.01 126.49) (width 0.3) (layer "B.Cu") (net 24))
 (segment (start 135.3525 126.9275) (end 135.3525 123.1025) (width 0.3) (layer "F.Cu") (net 23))
 (segment (start 137.25 128.825) (end 135.3525 126.9275) (width 0.3) (layer "F.Cu") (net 23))
 (via (at 135.3525 123.1025) (size 0.6) (drill 0.3) (layers "F.Cu" "B.Cu") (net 23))
 (segment (start 129.63 128.825) (end 135.3525 123.1025) (width 0.3) (layer "B.Cu") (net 23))
 (segment (start 135.3525 123.1025) (end 135.5 122.955) (width 0.3) (layer "B.Cu") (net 23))
 (segment (start 135.5 122.955) (end 135.5 90.165) (width 0.3) (layer "B.Cu") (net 23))
 (segment (start 135.5 90.165) (end 138.2 87.465) (width 0.3) (layer "B.Cu") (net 23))
 (segment (start 115.12 94.865) (end 112.8 92.545) (width 0.3) (layer "F.Cu") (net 20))
 (segment (start 115.12 116.855) (end 115.12 94.865) (width 0.3) (layer "F.Cu") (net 20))
 (segment (start 127.09 128.825) (end 115.12 116.855) (width 0.3) (layer "F.Cu") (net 20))
 (segment (start 144.87 128.825) (end 144.87 83.975) (width 0.3) (layer "B.Cu") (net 27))
 (segment (start 144.87 83.975) (end 138.2 77.305) (width 0.3) (layer "B.Cu") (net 27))
 (segment (start 141 85) (end 141 77.565) (width 0.3) (layer "F.Cu") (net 28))
 (segment (start 138.59 130.025) (end 139.79 128.825) (width 0.3) (layer "F.Cu") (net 28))
 (segment (start 125.75 130.025) (end 138.59 130.025) (width 0.3) (layer "F.Cu") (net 28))
 (segment (start 124.55 128.825) (end 125.75 130.025) (width 0.3) (layer "F.Cu") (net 28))
 (segment (start 141 77.565) (end 138.2 74.765) (width 0.3) (layer "F.Cu") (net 28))
 (via (at 141 85) (size 0.6) (drill 0.3) (layers "F.Cu" "B.Cu") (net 28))
 (segment (start 141.25 85.25) (end 141 85) (width 0.3) (layer "B.Cu") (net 28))
 (segment (start 141.25 127.365) (end 141.25 85.25) (width 0.3) (layer "B.Cu") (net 28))
 (segment (start 139.79 128.825) (end 141.25 127.365) (width 0.3) (layer "B.Cu") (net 28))
 (segment (start 142.33 83.975) (end 138.2 79.845) (width 0.3) (layer "B.Cu") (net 26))
 (segment (start 142.33 128.825) (end 142.33 83.975) (width 0.3) (layer "B.Cu") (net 26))
 (segment (start 143.75 53.75) (end 116.75 53.75) (width 0.3) (layer "B.Cu") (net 13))
 (segment (start 147.41 128.825) (end 147.41 57.41) (width 0.3) (layer "B.Cu") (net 13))
 (segment (start 116.75 70.815) (end 112.8 74.765) (width 0.3) (layer "B.Cu") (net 13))
 (segment (start 147.41 57.41) (end 143.75 53.75) (width 0.3) (layer "B.Cu") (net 13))
 (segment (start 116.75 53.75) (end 116.75 70.815) (width 0.3) (layer "B.Cu") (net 13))
 (segment (start 116.44 70.785) (end 112.8 67.145) (width 0.3) (layer "F.Cu") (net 10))
 (segment (start 134.71 128.825) (end 116.44 110.555) (width 0.3) (layer "F.Cu") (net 10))
 (segment (start 116.44 110.555) (end 116.44 70.785) (width 0.3) (layer "F.Cu") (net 10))
 (segment (start 136 115.925) (end 150.75 101.175) (width 0.5) (layer "F.Cu") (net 1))
 (segment (start 135.45 115.925) (end 136 115.925) (width 0.5) (layer "F.Cu") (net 1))
 (segment (start 150.75 101.175) (end 150.75 87.8) (width 0.5) (layer "F.Cu") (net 1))
 (segment (start 137.77 108.925) (end 148.75 97.945) (width 0.5) (layer "F.Cu") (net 2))
 (segment (start 135.45 108.925) (end 137.77 108.925) (width 0.5) (layer "F.Cu") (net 2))
 (segment (start 148.75 97.945) (end 148.75 87.8) (width 0.5) (layer "F.Cu") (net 2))
 (segment (start 132.5 103.5) (end 135 101) (width 0.5) (layer "F.Cu") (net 5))
 (segment (start 132.5 116.625) (end 132.5 103.5) (width 0.5) (layer "F.Cu") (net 5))
 (segment (start 135 60.185) (end 138.2 56.985) (width 0.5) (layer "F.Cu") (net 5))
 (segment (start 135 101) (end 135 60.185) (width 0.5) (layer "F.Cu") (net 5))
 (segment (start 135.45 119.575) (end 132.5 116.625) (width 0.5) (layer "F.Cu") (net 5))
 (via (at 137 56.75) (size 0.6) (drill 0.3) (layers "F.Cu" "B.Cu") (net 5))
 (segment (start 137 56.75) (end 137.015 56.735) (width 0.5) (layer "B.Cu") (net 5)))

